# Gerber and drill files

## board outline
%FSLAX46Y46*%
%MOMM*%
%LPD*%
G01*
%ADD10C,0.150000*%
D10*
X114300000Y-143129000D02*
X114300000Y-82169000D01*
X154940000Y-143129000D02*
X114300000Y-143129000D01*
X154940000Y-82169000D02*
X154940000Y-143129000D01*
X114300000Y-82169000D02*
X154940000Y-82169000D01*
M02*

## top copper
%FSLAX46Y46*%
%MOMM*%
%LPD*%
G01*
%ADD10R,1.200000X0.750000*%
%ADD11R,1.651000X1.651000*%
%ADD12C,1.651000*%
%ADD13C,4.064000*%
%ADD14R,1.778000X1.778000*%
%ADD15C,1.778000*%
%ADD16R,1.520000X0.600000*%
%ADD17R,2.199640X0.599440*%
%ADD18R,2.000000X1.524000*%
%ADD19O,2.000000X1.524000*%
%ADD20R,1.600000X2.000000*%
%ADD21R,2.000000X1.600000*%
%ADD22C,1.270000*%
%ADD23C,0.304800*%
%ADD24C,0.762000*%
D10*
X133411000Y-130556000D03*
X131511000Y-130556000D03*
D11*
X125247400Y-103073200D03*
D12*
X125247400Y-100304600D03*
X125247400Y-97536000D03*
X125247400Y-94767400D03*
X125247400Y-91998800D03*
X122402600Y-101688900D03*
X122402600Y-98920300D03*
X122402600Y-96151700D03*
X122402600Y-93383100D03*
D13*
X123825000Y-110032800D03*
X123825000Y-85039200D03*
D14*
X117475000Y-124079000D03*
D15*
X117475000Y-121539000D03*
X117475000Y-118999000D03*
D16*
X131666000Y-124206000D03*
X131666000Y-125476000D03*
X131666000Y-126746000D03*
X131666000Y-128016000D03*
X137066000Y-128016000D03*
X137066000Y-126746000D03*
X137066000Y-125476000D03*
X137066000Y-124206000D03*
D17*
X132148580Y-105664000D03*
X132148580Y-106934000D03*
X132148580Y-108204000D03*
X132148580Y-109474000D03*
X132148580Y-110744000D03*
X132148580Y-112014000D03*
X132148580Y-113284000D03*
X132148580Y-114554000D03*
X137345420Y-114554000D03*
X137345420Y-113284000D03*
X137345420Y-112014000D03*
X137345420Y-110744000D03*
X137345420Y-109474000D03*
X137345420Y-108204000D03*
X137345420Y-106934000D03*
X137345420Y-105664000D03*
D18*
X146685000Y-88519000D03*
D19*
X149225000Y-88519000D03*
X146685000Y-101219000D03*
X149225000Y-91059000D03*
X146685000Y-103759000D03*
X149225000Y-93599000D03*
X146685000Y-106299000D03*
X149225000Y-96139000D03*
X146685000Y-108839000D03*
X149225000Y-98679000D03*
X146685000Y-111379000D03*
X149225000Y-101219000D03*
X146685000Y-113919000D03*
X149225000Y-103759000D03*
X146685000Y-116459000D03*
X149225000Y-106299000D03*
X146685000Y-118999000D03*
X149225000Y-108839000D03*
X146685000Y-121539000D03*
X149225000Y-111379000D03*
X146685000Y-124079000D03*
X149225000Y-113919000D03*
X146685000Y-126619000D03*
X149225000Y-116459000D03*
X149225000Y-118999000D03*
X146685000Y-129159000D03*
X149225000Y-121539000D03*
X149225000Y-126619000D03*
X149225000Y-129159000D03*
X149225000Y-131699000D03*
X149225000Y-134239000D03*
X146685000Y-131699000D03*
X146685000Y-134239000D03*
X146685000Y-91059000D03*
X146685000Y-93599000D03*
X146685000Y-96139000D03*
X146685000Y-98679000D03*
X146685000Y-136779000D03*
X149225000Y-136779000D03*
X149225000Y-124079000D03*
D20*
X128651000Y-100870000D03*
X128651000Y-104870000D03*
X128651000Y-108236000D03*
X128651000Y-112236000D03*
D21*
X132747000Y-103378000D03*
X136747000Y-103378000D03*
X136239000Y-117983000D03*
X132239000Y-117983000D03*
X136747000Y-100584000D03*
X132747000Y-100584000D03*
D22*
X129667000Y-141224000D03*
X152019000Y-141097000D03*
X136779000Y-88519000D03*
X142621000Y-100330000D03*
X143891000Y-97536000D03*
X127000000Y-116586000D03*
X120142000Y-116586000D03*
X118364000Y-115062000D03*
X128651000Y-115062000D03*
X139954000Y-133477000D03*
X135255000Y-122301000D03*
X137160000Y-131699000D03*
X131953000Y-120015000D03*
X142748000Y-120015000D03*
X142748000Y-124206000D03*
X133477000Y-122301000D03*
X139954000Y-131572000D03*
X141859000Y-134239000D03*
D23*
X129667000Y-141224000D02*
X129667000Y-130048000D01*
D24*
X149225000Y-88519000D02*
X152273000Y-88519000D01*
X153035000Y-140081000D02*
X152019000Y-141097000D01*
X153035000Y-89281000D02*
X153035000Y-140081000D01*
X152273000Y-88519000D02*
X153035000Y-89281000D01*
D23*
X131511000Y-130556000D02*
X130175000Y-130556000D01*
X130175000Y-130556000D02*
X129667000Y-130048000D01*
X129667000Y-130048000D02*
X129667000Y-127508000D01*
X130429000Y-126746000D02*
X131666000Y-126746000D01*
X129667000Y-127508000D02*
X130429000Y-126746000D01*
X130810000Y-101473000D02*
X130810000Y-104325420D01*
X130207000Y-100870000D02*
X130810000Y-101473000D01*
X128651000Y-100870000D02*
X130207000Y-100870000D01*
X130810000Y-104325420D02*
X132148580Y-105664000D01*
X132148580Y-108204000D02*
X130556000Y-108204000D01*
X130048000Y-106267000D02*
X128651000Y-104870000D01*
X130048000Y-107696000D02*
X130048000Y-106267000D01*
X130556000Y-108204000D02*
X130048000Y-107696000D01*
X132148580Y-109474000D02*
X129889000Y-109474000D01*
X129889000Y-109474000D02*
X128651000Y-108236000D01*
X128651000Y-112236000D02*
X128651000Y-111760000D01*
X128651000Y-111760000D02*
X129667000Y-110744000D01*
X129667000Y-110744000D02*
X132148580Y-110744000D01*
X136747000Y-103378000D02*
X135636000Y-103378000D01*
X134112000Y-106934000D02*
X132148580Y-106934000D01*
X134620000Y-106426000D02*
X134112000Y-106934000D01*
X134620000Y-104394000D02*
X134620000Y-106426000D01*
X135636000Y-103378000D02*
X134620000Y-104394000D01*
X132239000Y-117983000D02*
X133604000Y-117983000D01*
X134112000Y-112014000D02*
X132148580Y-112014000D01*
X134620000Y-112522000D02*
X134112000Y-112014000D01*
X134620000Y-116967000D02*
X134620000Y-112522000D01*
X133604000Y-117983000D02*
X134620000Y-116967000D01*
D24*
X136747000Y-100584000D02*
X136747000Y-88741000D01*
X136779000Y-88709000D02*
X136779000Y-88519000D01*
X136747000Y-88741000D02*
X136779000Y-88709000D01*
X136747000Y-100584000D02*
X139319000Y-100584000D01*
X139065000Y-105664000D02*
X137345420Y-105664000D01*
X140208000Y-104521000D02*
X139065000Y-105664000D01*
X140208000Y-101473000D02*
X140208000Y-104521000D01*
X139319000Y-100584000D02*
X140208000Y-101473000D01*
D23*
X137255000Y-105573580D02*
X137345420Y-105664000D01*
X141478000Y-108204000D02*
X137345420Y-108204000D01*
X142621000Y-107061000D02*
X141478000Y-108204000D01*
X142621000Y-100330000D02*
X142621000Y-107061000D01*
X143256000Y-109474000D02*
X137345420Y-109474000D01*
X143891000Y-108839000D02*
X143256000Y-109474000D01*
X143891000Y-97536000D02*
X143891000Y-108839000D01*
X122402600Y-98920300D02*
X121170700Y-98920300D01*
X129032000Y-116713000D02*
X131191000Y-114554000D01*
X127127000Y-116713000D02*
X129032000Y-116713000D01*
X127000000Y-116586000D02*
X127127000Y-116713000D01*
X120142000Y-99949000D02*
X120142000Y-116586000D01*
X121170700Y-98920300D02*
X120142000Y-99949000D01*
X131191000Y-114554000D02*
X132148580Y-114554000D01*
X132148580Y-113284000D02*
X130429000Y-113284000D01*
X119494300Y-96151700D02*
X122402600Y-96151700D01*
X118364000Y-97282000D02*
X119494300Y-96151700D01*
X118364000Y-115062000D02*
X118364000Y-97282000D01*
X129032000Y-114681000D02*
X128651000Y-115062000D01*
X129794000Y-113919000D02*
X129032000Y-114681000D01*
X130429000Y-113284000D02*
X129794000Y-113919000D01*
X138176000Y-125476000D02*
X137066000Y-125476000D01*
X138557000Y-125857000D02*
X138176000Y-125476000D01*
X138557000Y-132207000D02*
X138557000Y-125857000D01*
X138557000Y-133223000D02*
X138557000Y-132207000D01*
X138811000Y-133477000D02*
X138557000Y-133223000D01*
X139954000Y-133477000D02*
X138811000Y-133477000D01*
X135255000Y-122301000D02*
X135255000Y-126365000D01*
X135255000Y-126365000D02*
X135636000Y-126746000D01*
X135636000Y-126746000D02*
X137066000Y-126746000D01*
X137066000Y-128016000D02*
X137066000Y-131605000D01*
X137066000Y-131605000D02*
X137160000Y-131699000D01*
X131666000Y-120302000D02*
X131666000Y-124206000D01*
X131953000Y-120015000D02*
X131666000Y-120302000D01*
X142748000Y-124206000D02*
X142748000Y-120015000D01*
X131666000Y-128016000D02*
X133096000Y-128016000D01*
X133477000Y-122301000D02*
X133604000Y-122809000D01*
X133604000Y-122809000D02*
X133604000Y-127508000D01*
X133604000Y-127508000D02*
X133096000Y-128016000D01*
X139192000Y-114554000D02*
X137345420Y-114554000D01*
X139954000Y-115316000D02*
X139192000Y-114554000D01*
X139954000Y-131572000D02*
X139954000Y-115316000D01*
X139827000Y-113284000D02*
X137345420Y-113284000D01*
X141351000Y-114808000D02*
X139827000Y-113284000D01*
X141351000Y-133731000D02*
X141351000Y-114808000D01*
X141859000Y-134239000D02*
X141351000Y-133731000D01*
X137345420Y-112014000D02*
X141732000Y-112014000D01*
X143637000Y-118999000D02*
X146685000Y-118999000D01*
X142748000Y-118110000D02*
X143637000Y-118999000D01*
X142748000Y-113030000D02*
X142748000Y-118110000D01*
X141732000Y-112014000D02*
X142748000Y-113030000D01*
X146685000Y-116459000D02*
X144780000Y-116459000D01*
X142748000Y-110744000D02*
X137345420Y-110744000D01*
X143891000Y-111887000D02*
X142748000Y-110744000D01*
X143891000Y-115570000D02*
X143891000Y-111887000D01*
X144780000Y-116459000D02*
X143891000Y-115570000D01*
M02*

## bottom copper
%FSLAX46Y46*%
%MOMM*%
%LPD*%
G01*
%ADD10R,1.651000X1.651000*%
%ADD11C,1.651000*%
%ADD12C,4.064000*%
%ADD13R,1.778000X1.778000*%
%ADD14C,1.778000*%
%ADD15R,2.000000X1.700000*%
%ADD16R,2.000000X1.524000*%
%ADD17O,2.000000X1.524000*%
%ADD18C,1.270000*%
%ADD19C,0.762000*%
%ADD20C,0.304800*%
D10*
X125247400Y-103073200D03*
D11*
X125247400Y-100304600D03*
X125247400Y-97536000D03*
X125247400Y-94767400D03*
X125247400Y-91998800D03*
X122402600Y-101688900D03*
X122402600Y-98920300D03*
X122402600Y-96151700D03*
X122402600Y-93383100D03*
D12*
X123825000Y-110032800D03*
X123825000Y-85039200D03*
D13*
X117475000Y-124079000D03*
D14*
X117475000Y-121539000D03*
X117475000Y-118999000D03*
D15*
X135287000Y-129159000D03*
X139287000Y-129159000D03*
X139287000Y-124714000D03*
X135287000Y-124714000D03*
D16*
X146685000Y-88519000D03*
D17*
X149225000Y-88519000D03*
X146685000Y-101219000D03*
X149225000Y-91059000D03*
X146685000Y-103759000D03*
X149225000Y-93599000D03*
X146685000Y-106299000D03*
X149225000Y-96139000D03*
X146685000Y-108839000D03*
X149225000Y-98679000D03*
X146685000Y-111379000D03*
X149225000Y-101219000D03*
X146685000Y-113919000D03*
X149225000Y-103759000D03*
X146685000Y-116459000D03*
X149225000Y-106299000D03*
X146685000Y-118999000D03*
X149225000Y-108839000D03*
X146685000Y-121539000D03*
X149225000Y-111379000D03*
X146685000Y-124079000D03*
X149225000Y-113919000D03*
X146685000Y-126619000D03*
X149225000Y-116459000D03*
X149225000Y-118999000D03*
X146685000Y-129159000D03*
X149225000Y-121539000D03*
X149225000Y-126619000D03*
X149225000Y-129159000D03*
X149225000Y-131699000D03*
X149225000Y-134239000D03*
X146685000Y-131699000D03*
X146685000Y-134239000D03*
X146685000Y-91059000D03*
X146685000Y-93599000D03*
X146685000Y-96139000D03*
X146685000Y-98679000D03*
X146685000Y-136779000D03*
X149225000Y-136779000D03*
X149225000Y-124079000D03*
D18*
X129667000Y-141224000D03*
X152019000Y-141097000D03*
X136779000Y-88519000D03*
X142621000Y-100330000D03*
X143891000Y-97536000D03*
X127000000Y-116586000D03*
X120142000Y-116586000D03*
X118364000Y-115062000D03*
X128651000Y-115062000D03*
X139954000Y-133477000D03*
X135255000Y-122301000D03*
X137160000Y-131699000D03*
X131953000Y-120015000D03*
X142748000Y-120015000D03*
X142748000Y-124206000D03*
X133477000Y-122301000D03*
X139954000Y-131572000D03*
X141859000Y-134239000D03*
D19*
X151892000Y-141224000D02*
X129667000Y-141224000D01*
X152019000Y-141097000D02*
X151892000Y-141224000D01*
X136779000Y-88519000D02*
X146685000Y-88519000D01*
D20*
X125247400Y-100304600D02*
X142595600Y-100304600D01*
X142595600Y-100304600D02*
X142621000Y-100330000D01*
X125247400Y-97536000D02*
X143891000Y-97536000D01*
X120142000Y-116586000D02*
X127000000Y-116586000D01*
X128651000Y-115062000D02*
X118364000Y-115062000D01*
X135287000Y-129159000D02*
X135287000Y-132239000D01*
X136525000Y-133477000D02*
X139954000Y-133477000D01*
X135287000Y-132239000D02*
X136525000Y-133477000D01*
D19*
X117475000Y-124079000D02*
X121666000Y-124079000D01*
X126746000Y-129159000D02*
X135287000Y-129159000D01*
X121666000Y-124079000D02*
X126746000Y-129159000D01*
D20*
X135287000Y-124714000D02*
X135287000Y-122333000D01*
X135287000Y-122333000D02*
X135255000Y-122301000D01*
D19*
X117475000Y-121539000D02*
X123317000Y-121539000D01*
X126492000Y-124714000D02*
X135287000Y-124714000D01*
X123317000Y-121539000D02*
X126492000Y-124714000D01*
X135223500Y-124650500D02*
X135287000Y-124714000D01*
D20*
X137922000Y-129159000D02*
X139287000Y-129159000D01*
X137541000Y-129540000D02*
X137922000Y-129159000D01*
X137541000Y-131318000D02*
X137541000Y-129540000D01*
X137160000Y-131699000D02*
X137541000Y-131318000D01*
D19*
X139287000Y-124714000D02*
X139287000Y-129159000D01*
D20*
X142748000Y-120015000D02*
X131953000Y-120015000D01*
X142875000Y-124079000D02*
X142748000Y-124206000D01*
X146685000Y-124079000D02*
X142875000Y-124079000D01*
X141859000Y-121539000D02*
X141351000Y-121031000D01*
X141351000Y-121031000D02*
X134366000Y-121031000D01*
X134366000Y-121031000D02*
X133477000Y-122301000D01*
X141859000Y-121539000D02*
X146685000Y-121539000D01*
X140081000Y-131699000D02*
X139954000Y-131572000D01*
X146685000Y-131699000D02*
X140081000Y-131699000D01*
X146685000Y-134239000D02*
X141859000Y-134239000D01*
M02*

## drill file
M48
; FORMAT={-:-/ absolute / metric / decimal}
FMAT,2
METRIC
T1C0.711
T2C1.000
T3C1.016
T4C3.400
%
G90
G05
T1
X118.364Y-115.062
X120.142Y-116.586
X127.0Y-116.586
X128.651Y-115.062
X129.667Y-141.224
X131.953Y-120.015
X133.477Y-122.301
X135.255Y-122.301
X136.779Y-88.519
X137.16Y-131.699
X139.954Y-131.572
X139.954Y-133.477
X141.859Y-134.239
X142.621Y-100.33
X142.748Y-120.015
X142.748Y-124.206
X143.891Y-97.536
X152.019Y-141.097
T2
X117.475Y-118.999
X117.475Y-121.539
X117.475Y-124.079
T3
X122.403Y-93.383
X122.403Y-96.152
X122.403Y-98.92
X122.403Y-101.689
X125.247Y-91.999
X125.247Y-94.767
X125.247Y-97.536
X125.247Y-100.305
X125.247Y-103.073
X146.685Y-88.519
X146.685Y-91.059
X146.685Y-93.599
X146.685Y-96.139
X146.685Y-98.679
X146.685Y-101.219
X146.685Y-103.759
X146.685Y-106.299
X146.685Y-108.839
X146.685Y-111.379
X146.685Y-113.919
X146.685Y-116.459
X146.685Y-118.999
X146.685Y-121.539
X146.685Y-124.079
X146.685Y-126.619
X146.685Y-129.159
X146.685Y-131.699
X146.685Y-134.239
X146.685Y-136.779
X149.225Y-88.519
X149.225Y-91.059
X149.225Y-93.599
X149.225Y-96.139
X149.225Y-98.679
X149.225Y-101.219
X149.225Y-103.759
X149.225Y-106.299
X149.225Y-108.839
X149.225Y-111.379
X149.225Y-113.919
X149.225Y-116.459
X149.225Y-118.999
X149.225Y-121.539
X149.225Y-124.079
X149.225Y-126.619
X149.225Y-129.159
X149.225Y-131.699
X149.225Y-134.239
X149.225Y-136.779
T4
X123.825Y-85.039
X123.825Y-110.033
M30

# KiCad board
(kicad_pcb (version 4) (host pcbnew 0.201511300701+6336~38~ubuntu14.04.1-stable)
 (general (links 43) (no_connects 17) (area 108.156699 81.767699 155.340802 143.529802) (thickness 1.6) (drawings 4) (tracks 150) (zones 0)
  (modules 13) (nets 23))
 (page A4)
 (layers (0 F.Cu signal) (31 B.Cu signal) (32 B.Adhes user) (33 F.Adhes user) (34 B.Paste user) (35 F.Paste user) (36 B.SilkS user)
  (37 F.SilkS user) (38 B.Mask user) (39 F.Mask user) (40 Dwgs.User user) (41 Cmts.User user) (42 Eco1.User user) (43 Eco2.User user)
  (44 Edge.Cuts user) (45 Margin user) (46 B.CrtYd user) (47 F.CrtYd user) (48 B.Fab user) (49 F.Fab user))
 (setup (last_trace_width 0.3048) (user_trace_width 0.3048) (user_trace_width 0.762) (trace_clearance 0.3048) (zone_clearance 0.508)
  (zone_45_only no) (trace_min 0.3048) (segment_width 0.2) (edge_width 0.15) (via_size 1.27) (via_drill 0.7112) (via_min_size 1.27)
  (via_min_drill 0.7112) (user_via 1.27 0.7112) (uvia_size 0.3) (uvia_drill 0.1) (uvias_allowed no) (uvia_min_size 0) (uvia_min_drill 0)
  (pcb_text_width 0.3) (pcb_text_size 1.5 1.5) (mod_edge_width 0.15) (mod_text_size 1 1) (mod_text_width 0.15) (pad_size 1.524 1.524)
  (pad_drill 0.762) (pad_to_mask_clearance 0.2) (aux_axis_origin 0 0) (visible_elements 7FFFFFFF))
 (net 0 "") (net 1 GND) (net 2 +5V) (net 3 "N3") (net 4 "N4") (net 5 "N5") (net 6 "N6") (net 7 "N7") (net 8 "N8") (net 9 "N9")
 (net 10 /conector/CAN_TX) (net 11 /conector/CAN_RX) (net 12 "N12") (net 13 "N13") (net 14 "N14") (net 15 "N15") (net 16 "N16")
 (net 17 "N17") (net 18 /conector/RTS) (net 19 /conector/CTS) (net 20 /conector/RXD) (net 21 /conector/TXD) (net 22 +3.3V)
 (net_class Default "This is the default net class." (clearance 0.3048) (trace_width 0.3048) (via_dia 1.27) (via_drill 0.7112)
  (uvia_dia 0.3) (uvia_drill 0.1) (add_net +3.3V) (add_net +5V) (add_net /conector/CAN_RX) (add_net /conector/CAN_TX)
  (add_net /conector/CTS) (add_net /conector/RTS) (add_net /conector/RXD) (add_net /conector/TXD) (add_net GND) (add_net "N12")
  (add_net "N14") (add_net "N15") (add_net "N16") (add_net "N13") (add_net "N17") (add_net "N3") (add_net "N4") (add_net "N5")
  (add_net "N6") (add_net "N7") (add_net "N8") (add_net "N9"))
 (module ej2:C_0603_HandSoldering (layer F.Cu) (at 132.461 130.556 180)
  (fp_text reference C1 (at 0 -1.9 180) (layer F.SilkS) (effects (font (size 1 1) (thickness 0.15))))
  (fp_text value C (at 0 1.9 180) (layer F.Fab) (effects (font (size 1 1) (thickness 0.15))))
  (pad 1 smd rect (at -0.95 0 180) (size 1.2 0.75) (layers F.Cu F.Paste F.Mask) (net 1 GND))
  (pad 2 smd rect (at 0.95 0 180) (size 1.2 0.75) (layers F.Cu F.Paste F.Mask) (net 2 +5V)))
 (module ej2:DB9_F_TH (layer F.Cu) (at 123.825 97.536 90)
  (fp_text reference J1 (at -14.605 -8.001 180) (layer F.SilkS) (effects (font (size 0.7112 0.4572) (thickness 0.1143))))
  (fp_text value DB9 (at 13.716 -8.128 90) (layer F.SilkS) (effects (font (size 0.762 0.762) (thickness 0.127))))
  (pad 1 thru_hole rect (at -5.5372 1.4224 90) (size 1.651 1.651) (drill 1.016) (layers *.Cu *.Mask))
  (pad 2 thru_hole circle (at -2.7686 1.4224 90) (size 1.651 1.651) (drill 1.016) (layers *.Cu *.Mask) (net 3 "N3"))
  (pad 3 thru_hole circle (at 0 1.4224 90) (size 1.651 1.651) (drill 1.016) (layers *.Cu *.Mask) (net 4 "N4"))
  (pad 4 thru_hole circle (at 2.7686 1.4224 90) (size 1.651 1.651) (drill 1.016) (layers *.Cu *.Mask))
  (pad 5 thru_hole circle (at 5.5372 1.4224 90) (size 1.651 1.651) (drill 1.016) (layers *.Cu *.Mask))
  (pad 6 thru_hole circle (at -4.1529 -1.4224 90) (size 1.651 1.651) (drill 1.016) (layers *.Cu *.Mask))
  (pad 7 thru_hole circle (at -1.3843 -1.4224 90) (size 1.651 1.651) (drill 1.016) (layers *.Cu *.Mask) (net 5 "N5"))
  (pad 8 thru_hole circle (at 1.3843 -1.4224 90) (size 1.651 1.651) (drill 1.016) (layers *.Cu *.Mask) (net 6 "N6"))
  (pad 9 thru_hole circle (at 4.1529 -1.4224 90) (size 1.651 1.651) (drill 1.016) (layers *.Cu *.Mask))
  (pad 10 thru_hole circle (at -12.4968 0 90) (size 4.064 4.064) (drill 3.4) (layers *.Cu *.Mask))
  (pad 11 thru_hole circle (at 12.4968 0 90) (size 4.064 4.064) (drill 3.4) (layers *.Cu *.Mask)))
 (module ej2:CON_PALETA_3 (layer F.Cu) (at 117.475 121.539 90)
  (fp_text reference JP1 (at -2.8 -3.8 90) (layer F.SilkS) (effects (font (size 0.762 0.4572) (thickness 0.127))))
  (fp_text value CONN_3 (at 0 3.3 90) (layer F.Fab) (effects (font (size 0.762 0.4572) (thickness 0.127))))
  (pad 1 thru_hole rect (at -2.54 0 90) (size 1.778 1.778) (drill 1) (layers *.Cu *.Mask) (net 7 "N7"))
  (pad 2 thru_hole circle (at 0 0 90) (size 1.778 1.778) (drill 1) (layers *.Cu *.Mask) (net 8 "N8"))
  (pad 3 thru_hole circle (at 2.54 0 90) (size 1.778 1.778) (drill 1) (layers *.Cu *.Mask) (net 1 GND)))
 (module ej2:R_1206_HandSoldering (layer B.Cu) (at 137.287 129.159)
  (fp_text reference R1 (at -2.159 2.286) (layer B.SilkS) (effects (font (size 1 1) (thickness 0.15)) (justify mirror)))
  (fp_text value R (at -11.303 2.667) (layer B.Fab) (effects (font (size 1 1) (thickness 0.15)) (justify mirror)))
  (pad 1 smd rect (at -2 0) (size 2 1.7) (layers B.Cu B.Paste B.Mask) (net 7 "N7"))
  (pad 2 smd rect (at 2 0) (size 2 1.7) (layers B.Cu B.Paste B.Mask) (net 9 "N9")))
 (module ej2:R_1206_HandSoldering (layer B.Cu) (at 137.287 124.714 180)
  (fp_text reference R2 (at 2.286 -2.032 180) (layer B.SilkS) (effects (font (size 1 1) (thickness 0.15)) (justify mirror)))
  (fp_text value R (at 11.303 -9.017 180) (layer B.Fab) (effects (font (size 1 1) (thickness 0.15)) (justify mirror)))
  (pad 1 smd rect (at -2 0 180) (size 2 1.7) (layers B.Cu B.Paste B.Mask) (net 9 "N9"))
  (pad 2 smd rect (at 2 0 180) (size 2 1.7) (layers B.Cu B.Paste B.Mask) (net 8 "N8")))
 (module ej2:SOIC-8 (layer F.Cu) (at 134.366 126.111)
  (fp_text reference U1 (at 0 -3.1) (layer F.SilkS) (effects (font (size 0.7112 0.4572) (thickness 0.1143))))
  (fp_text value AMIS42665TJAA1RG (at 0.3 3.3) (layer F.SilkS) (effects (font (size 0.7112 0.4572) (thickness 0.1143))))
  (pad 1 smd rect (at -2.7 -1.905 270) (size 0.6 1.52) (layers F.Cu F.Paste F.Mask) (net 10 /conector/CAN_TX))
  (pad 2 smd rect (at -2.7 -0.635 270) (size 0.6 1.52) (layers F.Cu F.Paste F.Mask) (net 1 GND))
  (pad 3 smd rect (at -2.7 0.635 270) (size 0.6 1.52) (layers F.Cu F.Paste F.Mask) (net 2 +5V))
  (pad 4 smd rect (at -2.7 1.905 270) (size 0.6 1.52) (layers F.Cu F.Paste F.Mask) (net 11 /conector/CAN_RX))
  (pad 5 smd rect (at 2.7 1.905 270) (size 0.6 1.52) (layers F.Cu F.Paste F.Mask) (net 9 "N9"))
  (pad 6 smd rect (at 2.7 0.635 270) (size 0.6 1.52) (layers F.Cu F.Paste F.Mask) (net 8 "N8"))
  (pad 7 smd rect (at 2.7 -0.635 270) (size 0.6 1.52) (layers F.Cu F.Paste F.Mask) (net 7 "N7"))
  (pad 8 smd rect (at 2.7 -1.905 270) (size 0.6 1.52) (layers F.Cu F.Paste F.Mask) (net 1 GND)))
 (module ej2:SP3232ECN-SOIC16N (layer F.Cu) (at 134.747 110.109 270)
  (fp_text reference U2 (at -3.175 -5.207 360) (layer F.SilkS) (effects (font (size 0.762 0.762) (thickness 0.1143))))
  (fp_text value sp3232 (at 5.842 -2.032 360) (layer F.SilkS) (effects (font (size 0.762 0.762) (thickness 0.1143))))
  (pad 1 smd rect (at -4.445 2.59842 270) (size 0.59944 2.19964) (layers F.Cu F.Paste F.Mask) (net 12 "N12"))
  (pad 2 smd rect (at -3.175 2.59842 270) (size 0.59944 2.19964) (layers F.Cu F.Paste F.Mask) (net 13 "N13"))
  (pad 3 smd rect (at -1.905 2.59842 270) (size 0.59944 2.19964) (layers F.Cu F.Paste F.Mask) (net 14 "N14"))
  (pad 4 smd rect (at -0.635 2.59842 270) (size 0.59944 2.19964) (layers F.Cu F.Paste F.Mask) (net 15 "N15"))
  (pad 5 smd rect (at 0.635 2.59842 270) (size 0.59944 2.19964) (layers F.Cu F.Paste F.Mask) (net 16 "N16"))
  (pad 6 smd rect (at 1.905 2.59842 270) (size 0.59944 2.19964) (layers F.Cu F.Paste F.Mask) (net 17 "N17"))
  (pad 7 smd rect (at 3.175 2.59842 270) (size 0.59944 2.19964) (layers F.Cu F.Paste F.Mask) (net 6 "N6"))
  (pad 8 smd rect (at 4.445 2.59842 270) (size 0.59944 2.19964) (layers F.Cu F.Paste F.Mask) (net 5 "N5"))
  (pad 9 smd rect (at 4.445 -2.59842 270) (size 0.59944 2.19964) (layers F.Cu F.Paste F.Mask) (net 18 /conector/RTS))
  (pad 10 smd rect (at 3.175 -2.59842 270) (size 0.59944 2.19964) (layers F.Cu F.Paste F.Mask) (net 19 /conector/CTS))
  (pad 11 smd rect (at 1.905 -2.59842 270) (size 0.59944 2.19964) (layers F.Cu F.Paste F.Mask) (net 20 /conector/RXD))
  (pad 12 smd rect (at 0.635 -2.59842 270) (size 0.59944 2.19964) (layers F.Cu F.Paste F.Mask) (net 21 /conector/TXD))
  (pad 13 smd rect (at -0.635 -2.59842 270) (size 0.59944 2.19964) (layers F.Cu F.Paste F.Mask) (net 4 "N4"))
  (pad 14 smd rect (at -1.905 -2.59842 270) (size 0.59944 2.19964) (layers F.Cu F.Paste F.Mask) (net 3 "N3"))
  (pad 15 smd rect (at -3.175 -2.59842 270) (size 0.59944 2.19964) (layers F.Cu F.Paste F.Mask) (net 1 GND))
  (pad 16 smd rect (at -4.445 -2.59842 270) (size 0.59944 2.19964) (layers F.Cu F.Paste F.Mask) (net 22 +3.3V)))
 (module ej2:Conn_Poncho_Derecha (layer F.Cu) (at 146.685 88.519)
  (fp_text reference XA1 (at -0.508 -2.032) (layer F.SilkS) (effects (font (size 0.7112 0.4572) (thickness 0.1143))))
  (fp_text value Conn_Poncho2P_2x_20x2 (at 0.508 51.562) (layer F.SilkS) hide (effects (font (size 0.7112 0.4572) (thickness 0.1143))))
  (pad 1 thru_hole rect (at 0 0 270) (size 1.524 2) (drill 1.016) (layers *.Cu *.Mask) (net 22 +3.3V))
  (pad 2 thru_hole oval (at 2.54 0 270) (size 1.524 2) (drill 1.016) (layers *.Cu *.Mask) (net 2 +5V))
  (pad 11 thru_hole oval (at 0 12.7 270) (size 1.524 2) (drill 1.016) (layers *.Cu *.Mask))
  (pad 4 thru_hole oval (at 2.54 2.54 270) (size 1.524 2) (drill 1.016) (layers *.Cu *.Mask) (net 1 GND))
  (pad 13 thru_hole oval (at 0 15.24 270) (size 1.524 2) (drill 1.016) (layers *.Cu *.Mask))
  (pad 6 thru_hole oval (at 2.54 5.08 270) (size 1.524 2) (drill 1.016) (layers *.Cu *.Mask))
  (pad 15 thru_hole oval (at 0 17.78 270) (size 1.524 2) (drill 1.016) (layers *.Cu *.Mask))
  (pad 8 thru_hole oval (at 2.54 7.62 270) (size 1.524 2) (drill 1.016) (layers *.Cu *.Mask))
  (pad 17 thru_hole oval (at 0 20.32 270) (size 1.524 2) (drill 1.016) (layers *.Cu *.Mask))
  (pad 10 thru_hole oval (at 2.54 10.16 270) (size 1.524 2) (drill 1.016) (layers *.Cu *.Mask))
  (pad 19 thru_hole oval (at 0 22.86 270) (size 1.524 2) (drill 1.016) (layers *.Cu *.Mask))
  (pad 12 thru_hole oval (at 2.54 12.7 270) (size 1.524 2) (drill 1.016) (layers *.Cu *.Mask))
  (pad 21 thru_hole oval (at 0 25.4 270) (size 1.524 2) (drill 1.016) (layers *.Cu *.Mask))
  (pad 14 thru_hole oval (at 2.54 15.24 270) (size 1.524 2) (drill 1.016) (layers *.Cu *.Mask))
  (pad 23 thru_hole oval (at 0 27.94 270) (size 1.524 2) (drill 1.016) (layers *.Cu *.Mask) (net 21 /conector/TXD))
  (pad 16 thru_hole oval (at 2.54 17.78 270) (size 1.524 2) (drill 1.016) (layers *.Cu *.Mask))
  (pad 25 thru_hole oval (at 0 30.48 270) (size 1.524 2) (drill 1.016) (layers *.Cu *.Mask) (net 20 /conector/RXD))
  (pad 18 thru_hole oval (at 2.54 20.32 270) (size 1.524 2) (drill 1.016) (layers *.Cu *.Mask))
  (pad 27 thru_hole oval (at 0 33.02 270) (size 1.524 2) (drill 1.016) (layers *.Cu *.Mask) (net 11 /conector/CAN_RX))
  (pad 20 thru_hole oval (at 2.54 22.86 270) (size 1.524 2) (drill 1.016) (layers *.Cu *.Mask) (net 1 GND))
  (pad 29 thru_hole oval (at 0 35.56 270) (size 1.524 2) (drill 1.016) (layers *.Cu *.Mask) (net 10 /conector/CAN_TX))
  (pad 22 thru_hole oval (at 2.54 25.4 270) (size 1.524 2) (drill 1.016) (layers *.Cu *.Mask) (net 1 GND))
  (pad 31 thru_hole oval (at 0 38.1 270) (size 1.524 2) (drill 1.016) (layers *.Cu *.Mask))
  (pad 24 thru_hole oval (at 2.54 27.94 270) (size 1.524 2) (drill 1.016) (layers *.Cu *.Mask) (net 1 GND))
  (pad 26 thru_hole oval (at 2.54 30.48 270) (size 1.524 2) (drill 1.016) (layers *.Cu *.Mask) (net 1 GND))
  (pad 33 thru_hole oval (at 0 40.64 270) (size 1.524 2) (drill 1.016) (layers *.Cu *.Mask))
  (pad 28 thru_hole oval (at 2.54 33.02 270) (size 1.524 2) (drill 1.016) (layers *.Cu *.Mask) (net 1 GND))
  (pad 32 thru_hole oval (at 2.54 38.1 270) (size 1.524 2) (drill 1.016) (layers *.Cu *.Mask) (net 1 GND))
  (pad 34 thru_hole oval (at 2.54 40.64 270) (size 1.524 2) (drill 1.016) (layers *.Cu *.Mask))
  (pad 36 thru_hole oval (at 2.54 43.18 270) (size 1.524 2) (drill 1.016) (layers *.Cu *.Mask))
  (pad 38 thru_hole oval (at 2.54 45.72 270) (size 1.524 2) (drill 1.016) (layers *.Cu *.Mask) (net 1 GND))
  (pad 35 thru_hole oval (at 0 43.18 270) (size 1.524 2) (drill 1.016) (layers *.Cu *.Mask) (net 18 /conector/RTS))
  (pad 37 thru_hole oval (at 0 45.72 270) (size 1.524 2) (drill 1.016) (layers *.Cu *.Mask) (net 19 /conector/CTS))
  (pad 3 thru_hole oval (at 0 2.54 270) (size 1.524 2) (drill 1.016) (layers *.Cu *.Mask))
  (pad 5 thru_hole oval (at 0 5.08 270) (size 1.524 2) (drill 1.016) (layers *.Cu *.Mask))
  (pad 7 thru_hole oval (at 0 7.62 270) (size 1.524 2) (drill 1.016) (layers *.Cu *.Mask))
  (pad 9 thru_hole oval (at 0 10.16 270) (size 1.524 2) (drill 1.016) (layers *.Cu *.Mask))
  (pad 39 thru_hole oval (at 0 48.26 270) (size 1.524 2) (drill 1.016) (layers *.Cu *.Mask))
  (pad 40 thru_hole oval (at 2.54 48.26 270) (size 1.524 2) (drill 1.016) (layers *.Cu *.Mask) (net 1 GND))
  (pad 30 thru_hole oval (at 2.54 35.56 270) (size 1.524 2) (drill 1.016) (layers *.Cu *.Mask) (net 1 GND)))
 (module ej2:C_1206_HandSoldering (layer F.Cu) (at 128.651 102.87 270)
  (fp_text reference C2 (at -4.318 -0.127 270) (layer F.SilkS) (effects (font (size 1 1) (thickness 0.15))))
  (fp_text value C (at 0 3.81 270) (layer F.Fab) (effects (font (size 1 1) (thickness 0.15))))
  (pad 1 smd rect (at -2 0 270) (size 2 1.6) (layers F.Cu F.Paste F.Mask) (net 12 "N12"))
  (pad 2 smd rect (at 2 0 270) (size 2 1.6) (layers F.Cu F.Paste F.Mask) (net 14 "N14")))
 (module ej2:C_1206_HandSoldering (layer F.Cu) (at 128.651 110.236 270)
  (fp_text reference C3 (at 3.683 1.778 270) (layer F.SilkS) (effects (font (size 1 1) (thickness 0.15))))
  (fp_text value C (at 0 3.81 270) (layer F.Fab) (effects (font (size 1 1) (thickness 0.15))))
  (pad 1 smd rect (at -2 0 270) (size 2 1.6) (layers F.Cu F.Paste F.Mask) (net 15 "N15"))
  (pad 2 smd rect (at 2 0 270) (size 2 1.6) (layers F.Cu F.Paste F.Mask) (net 16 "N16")))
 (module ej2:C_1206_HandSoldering (layer F.Cu) (at 134.747 103.378)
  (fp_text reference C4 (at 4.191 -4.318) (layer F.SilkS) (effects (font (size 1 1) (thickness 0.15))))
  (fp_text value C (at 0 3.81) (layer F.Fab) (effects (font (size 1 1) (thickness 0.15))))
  (pad 1 smd rect (at -2 0) (size 2 1.6) (layers F.Cu F.Paste F.Mask) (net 1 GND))
  (pad 2 smd rect (at 2 0) (size 2 1.6) (layers F.Cu F.Paste F.Mask) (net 13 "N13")))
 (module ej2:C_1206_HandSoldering (layer F.Cu) (at 134.239 117.983 180)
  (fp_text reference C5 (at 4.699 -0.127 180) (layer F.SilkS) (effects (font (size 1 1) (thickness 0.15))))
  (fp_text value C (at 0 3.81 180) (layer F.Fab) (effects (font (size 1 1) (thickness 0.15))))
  (pad 1 smd rect (at -2 0 180) (size 2 1.6) (layers F.Cu F.Paste F.Mask) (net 1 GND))
  (pad 2 smd rect (at 2 0 180) (size 2 1.6) (layers F.Cu F.Paste F.Mask) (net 17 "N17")))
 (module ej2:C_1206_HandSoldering (layer F.Cu) (at 134.747 100.584 180)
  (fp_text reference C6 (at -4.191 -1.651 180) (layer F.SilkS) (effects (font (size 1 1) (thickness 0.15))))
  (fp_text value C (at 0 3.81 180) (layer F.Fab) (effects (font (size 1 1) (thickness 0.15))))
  (pad 1 smd rect (at -2 0 180) (size 2 1.6) (layers F.Cu F.Paste F.Mask) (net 22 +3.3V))
  (pad 2 smd rect (at 2 0 180) (size 2 1.6) (layers F.Cu F.Paste F.Mask) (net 1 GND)))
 (gr_line (start 114.3 143.129) (end 114.3 82.169) (angle 90) (layer Edge.Cuts) (width 0.15))
 (gr_line (start 154.94 143.129) (end 114.3 143.129) (angle 90) (layer Edge.Cuts) (width 0.15))
 (gr_line (start 154.94 82.169) (end 154.94 143.129) (angle 90) (layer Edge.Cuts) (width 0.15))
 (gr_line (start 114.3 82.169) (end 154.94 82.169) (angle 90) (layer Edge.Cuts) (width 0.15))
 (segment (start 129.667 141.224) (end 129.667 130.048) (width 0.3048) (layer F.Cu) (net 2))
 (segment (start 149.225 88.519) (end 152.273 88.519) (width 0.762) (layer F.Cu) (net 2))
 (via (at 129.667 141.224) (size 1.27) (drill 0.7112) (layers F.Cu B.Cu) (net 2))
 (segment (start 151.892 141.224) (end 129.667 141.224) (width 0.762) (layer B.Cu) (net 2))
 (segment (start 152.019 141.097) (end 151.892 141.224) (width 0.762) (layer B.Cu) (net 2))
 (via (at 152.019 141.097) (size 1.27) (drill 0.7112) (layers F.Cu B.Cu) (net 2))
 (segment (start 153.035 140.081) (end 152.019 141.097) (width 0.762) (layer F.Cu) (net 2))
 (segment (start 153.035 89.281) (end 153.035 140.081) (width 0.762) (layer F.Cu) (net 2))
 (segment (start 152.273 88.519) (end 153.035 89.281) (width 0.762) (layer F.Cu) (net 2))
 (segment (start 131.511 130.556) (end 130.175 130.556) (width 0.3048) (layer F.Cu) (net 2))
 (segment (start 130.175 130.556) (end 129.667 130.048) (width 0.3048) (layer F.Cu) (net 2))
 (segment (start 129.667 130.048) (end 129.667 127.508) (width 0.3048) (layer F.Cu) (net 2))
 (segment (start 130.429 126.746) (end 131.666 126.746) (width 0.3048) (layer F.Cu) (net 2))
 (segment (start 129.667 127.508) (end 130.429 126.746) (width 0.3048) (layer F.Cu) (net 2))
 (segment (start 130.81 101.473) (end 130.81 104.32542) (width 0.3048) (layer F.Cu) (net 12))
 (segment (start 130.207 100.87) (end 130.81 101.473) (width 0.3048) (layer F.Cu) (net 12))
 (segment (start 128.651 100.87) (end 130.207 100.87) (width 0.3048) (layer F.Cu) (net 12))
 (segment (start 130.81 104.32542) (end 132.14858 105.664) (width 0.3048) (layer F.Cu) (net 12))
 (segment (start 132.14858 108.204) (end 130.556 108.204) (width 0.3048) (layer F.Cu) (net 14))
 (segment (start 130.048 106.267) (end 128.651 104.87) (width 0.3048) (layer F.Cu) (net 14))
 (segment (start 130.048 107.696) (end 130.048 106.267) (width 0.3048) (layer F.Cu) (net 14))
 (segment (start 130.556 108.204) (end 130.048 107.696) (width 0.3048) (layer F.Cu) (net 14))
 (segment (start 132.14858 109.474) (end 129.889 109.474) (width 0.3048) (layer F.Cu) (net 15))
 (segment (start 129.889 109.474) (end 128.651 108.236) (width 0.3048) (layer F.Cu) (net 15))
 (segment (start 128.651 112.236) (end 128.651 111.76) (width 0.3048) (layer F.Cu) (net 16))
 (segment (start 128.651 111.76) (end 129.667 110.744) (width 0.3048) (layer F.Cu) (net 16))
 (segment (start 129.667 110.744) (end 132.14858 110.744) (width 0.3048) (layer F.Cu) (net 16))
 (segment (start 136.747 103.378) (end 135.636 103.378) (width 0.3048) (layer F.Cu) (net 13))
 (segment (start 134.112 106.934) (end 132.14858 106.934) (width 0.3048) (layer F.Cu) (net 13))
 (segment (start 134.62 106.426) (end 134.112 106.934) (width 0.3048) (layer F.Cu) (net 13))
 (segment (start 134.62 104.394) (end 134.62 106.426) (width 0.3048) (layer F.Cu) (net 13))
 (segment (start 135.636 103.378) (end 134.62 104.394) (width 0.3048) (layer F.Cu) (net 13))
 (segment (start 132.239 117.983) (end 133.604 117.983) (width 0.3048) (layer F.Cu) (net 17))
 (segment (start 134.112 112.014) (end 132.14858 112.014) (width 0.3048) (layer F.Cu) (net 17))
 (segment (start 134.62 112.522) (end 134.112 112.014) (width 0.3048) (layer F.Cu) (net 17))
 (segment (start 134.62 116.967) (end 134.62 112.522) (width 0.3048) (layer F.Cu) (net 17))
 (segment (start 133.604 117.983) (end 134.62 116.967) (width 0.3048) (layer F.Cu) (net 17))
 (segment (start 136.747 100.584) (end 136.747 88.741) (width 0.762) (layer F.Cu) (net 22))
 (segment (start 136.779 88.519) (end 146.685 88.519) (width 0.762) (layer B.Cu) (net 22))
 (via (at 136.779 88.519) (size 1.27) (drill 0.7112) (layers F.Cu B.Cu) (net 22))
 (segment (start 136.779 88.709) (end 136.779 88.519) (width 0.762) (layer F.Cu) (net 22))
 (segment (start 136.747 88.741) (end 136.779 88.709) (width 0.762) (layer F.Cu) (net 22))
 (segment (start 136.747 100.584) (end 139.319 100.584) (width 0.762) (layer F.Cu) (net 22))
 (segment (start 139.065 105.664) (end 137.34542 105.664) (width 0.762) (layer F.Cu) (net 22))
 (segment (start 140.208 104.521) (end 139.065 105.664) (width 0.762) (layer F.Cu) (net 22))
 (segment (start 140.208 101.473) (end 140.208 104.521) (width 0.762) (layer F.Cu) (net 22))
 (segment (start 139.319 100.584) (end 140.208 101.473) (width 0.762) (layer F.Cu) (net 22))
 (segment (start 137.255 105.57358) (end 137.34542 105.664) (width 0.3048) (layer F.Cu) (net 22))
 (segment (start 125.2474 100.3046) (end 142.5956 100.3046) (width 0.3048) (layer B.Cu) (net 3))
 (segment (start 141.478 108.204) (end 137.34542 108.204) (width 0.3048) (layer F.Cu) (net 3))
 (segment (start 142.621 107.061) (end 141.478 108.204) (width 0.3048) (layer F.Cu) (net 3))
 (segment (start 142.621 100.33) (end 142.621 107.061) (width 0.3048) (layer F.Cu) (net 3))
 (via (at 142.621 100.33) (size 1.27) (drill 0.7112) (layers F.Cu B.Cu) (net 3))
 (segment (start 142.5956 100.3046) (end 142.621 100.33) (width 0.3048) (layer B.Cu) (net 3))
 (segment (start 125.2474 97.536) (end 143.891 97.536) (width 0.3048) (layer B.Cu) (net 4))
 (segment (start 143.256 109.474) (end 137.34542 109.474) (width 0.3048) (layer F.Cu) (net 4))
 (segment (start 143.891 108.839) (end 143.256 109.474) (width 0.3048) (layer F.Cu) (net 4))
 (segment (start 143.891 97.536) (end 143.891 108.839) (width 0.3048) (layer F.Cu) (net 4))
 (via (at 143.891 97.536) (size 1.27) (drill 0.7112) (layers F.Cu B.Cu) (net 4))
 (segment (start 122.4026 98.9203) (end 121.1707 98.9203) (width 0.3048) (layer F.Cu) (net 5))
 (segment (start 129.032 116.713) (end 131.191 114.554) (width 0.3048) (layer F.Cu) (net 5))
 (segment (start 127.127 116.713) (end 129.032 116.713) (width 0.3048) (layer F.Cu) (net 5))
 (segment (start 127 116.586) (end 127.127 116.713) (width 0.3048) (layer F.Cu) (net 5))
 (via (at 127 116.586) (size 1.27) (drill 0.7112) (layers F.Cu B.Cu) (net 5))
 (segment (start 120.142 116.586) (end 127 116.586) (width 0.3048) (layer B.Cu) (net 5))
 (via (at 120.142 116.586) (size 1.27) (drill 0.7112) (layers F.Cu B.Cu) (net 5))
 (segment (start 120.142 99.949) (end 120.142 116.586) (width 0.3048) (layer F.Cu) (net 5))
 (segment (start 121.1707 98.9203) (end 120.142 99.949) (width 0.3048) (layer F.Cu) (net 5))
 (segment (start 131.191 114.554) (end 132.14858 114.554) (width 0.3048) (layer F.Cu) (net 5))
 (segment (start 132.14858 113.284) (end 130.429 113.284) (width 0.3048) (layer F.Cu) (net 6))
 (segment (start 119.4943 96.1517) (end 122.4026 96.1517) (width 0.3048) (layer F.Cu) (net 6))
 (segment (start 118.364 97.282) (end 119.4943 96.1517) (width 0.3048) (layer F.Cu) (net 6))
 (segment (start 118.364 115.062) (end 118.364 97.282) (width 0.3048) (layer F.Cu) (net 6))
 (via (at 118.364 115.062) (size 1.27) (drill 0.7112) (layers F.Cu B.Cu) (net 6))
 (segment (start 128.651 115.062) (end 118.364 115.062) (width 0.3048) (layer B.Cu) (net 6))
 (via (at 128.651 115.062) (size 1.27) (drill 0.7112) (layers F.Cu B.Cu) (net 6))
 (segment (start 129.032 114.681) (end 128.651 115.062) (width 0.3048) (layer F.Cu) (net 6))
 (segment (start 129.794 113.919) (end 129.032 114.681) (width 0.3048) (layer F.Cu) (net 6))
 (segment (start 130.429 113.284) (end 129.794 113.919) (width 0.3048) (layer F.Cu) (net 6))
 (segment (start 135.287 129.159) (end 135.287 132.239) (width 0.3048) (layer B.Cu) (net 7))
 (segment (start 138.176 125.476) (end 137.066 125.476) (width 0.3048) (layer F.Cu) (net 7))
 (segment (start 138.557 125.857) (end 138.176 125.476) (width 0.3048) (layer F.Cu) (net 7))
 (segment (start 138.557 132.207) (end 138.557 125.857) (width 0.3048) (layer F.Cu) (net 7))
 (segment (start 138.557 133.223) (end 138.557 132.207) (width 0.3048) (layer F.Cu) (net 7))
 (segment (start 138.811 133.477) (end 138.557 133.223) (width 0.3048) (layer F.Cu) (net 7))
 (segment (start 139.954 133.477) (end 138.811 133.477) (width 0.3048) (layer F.Cu) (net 7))
 (via (at 139.954 133.477) (size 1.27) (drill 0.7112) (layers F.Cu B.Cu) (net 7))
 (segment (start 136.525 133.477) (end 139.954 133.477) (width 0.3048) (layer B.Cu) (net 7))
 (segment (start 135.287 132.239) (end 136.525 133.477) (width 0.3048) (layer B.Cu) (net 7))
 (segment (start 117.475 124.079) (end 121.666 124.079) (width 0.762) (layer B.Cu) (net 7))
 (segment (start 126.746 129.159) (end 135.287 129.159) (width 0.762) (layer B.Cu) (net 7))
 (segment (start 121.666 124.079) (end 126.746 129.159) (width 0.762) (layer B.Cu) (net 7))
 (segment (start 135.287 124.714) (end 135.287 122.333) (width 0.3048) (layer B.Cu) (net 8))
 (segment (start 135.287 122.333) (end 135.255 122.301) (width 0.3048) (layer B.Cu) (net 8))
 (via (at 135.255 122.301) (size 1.27) (drill 0.7112) (layers F.Cu B.Cu) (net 8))
 (segment (start 135.255 122.301) (end 135.255 126.365) (width 0.3048) (layer F.Cu) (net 8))
 (segment (start 135.255 126.365) (end 135.636 126.746) (width 0.3048) (layer F.Cu) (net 8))
 (segment (start 135.636 126.746) (end 137.066 126.746) (width 0.3048) (layer F.Cu) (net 8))
 (segment (start 117.475 121.539) (end 123.317 121.539) (width 0.762) (layer B.Cu) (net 8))
 (segment (start 126.492 124.714) (end 135.287 124.714) (width 0.762) (layer B.Cu) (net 8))
 (segment (start 123.317 121.539) (end 126.492 124.714) (width 0.762) (layer B.Cu) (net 8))
 (segment (start 135.2235 124.6505) (end 135.287 124.714) (width 0.762) (layer B.Cu) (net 8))
 (segment (start 137.066 128.016) (end 137.066 131.605) (width 0.3048) (layer F.Cu) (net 9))
 (segment (start 137.922 129.159) (end 139.287 129.159) (width 0.3048) (layer B.Cu) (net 9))
 (segment (start 137.541 129.54) (end 137.922 129.159) (width 0.3048) (layer B.Cu) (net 9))
 (segment (start 137.541 131.318) (end 137.541 129.54) (width 0.3048) (layer B.Cu) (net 9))
 (segment (start 137.16 131.699) (end 137.541 131.318) (width 0.3048) (layer B.Cu) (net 9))
 (via (at 137.16 131.699) (size 1.27) (drill 0.7112) (layers F.Cu B.Cu) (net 9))
 (segment (start 137.066 131.605) (end 137.16 131.699) (width 0.3048) (layer F.Cu) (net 9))
 (segment (start 139.287 124.714) (end 139.287 129.159) (width 0.762) (layer B.Cu) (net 9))
 (segment (start 131.666 120.302) (end 131.666 124.206) (width 0.3048) (layer F.Cu) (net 10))
 (segment (start 131.953 120.015) (end 131.666 120.302) (width 0.3048) (layer F.Cu) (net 10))
 (via (at 131.953 120.015) (size 1.27) (drill 0.7112) (layers F.Cu B.Cu) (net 10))
 (segment (start 142.748 120.015) (end 131.953 120.015) (width 0.3048) (layer B.Cu) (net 10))
 (via (at 142.748 120.015) (size 1.27) (drill 0.7112) (layers F.Cu B.Cu) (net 10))
 (segment (start 142.748 124.206) (end 142.748 120.015) (width 0.3048) (layer F.Cu) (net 10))
 (via (at 142.748 124.206) (size 1.27) (drill 0.7112) (layers F.Cu B.Cu) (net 10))
 (segment (start 142.875 124.079) (end 142.748 124.206) (width 0.3048) (layer B.Cu) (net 10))
 (segment (start 146.685 124.079) (end 142.875 124.079) (width 0.3048) (layer B.Cu) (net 10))
 (segment (start 131.666 128.016) (end 133.096 128.016) (width 0.3048) (layer F.Cu) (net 11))
 (segment (start 141.859 121.539) (end 141.351 121.031) (width 0.3048) (layer B.Cu) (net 11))
 (segment (start 141.351 121.031) (end 134.366 121.031) (width 0.3048) (layer B.Cu) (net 11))
 (segment (start 134.366 121.031) (end 133.477 122.301) (width 0.3048) (layer B.Cu) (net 11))
 (via (at 133.477 122.301) (size 1.27) (drill 0.7112) (layers F.Cu B.Cu) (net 11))
 (segment (start 133.477 122.301) (end 133.604 122.809) (width 0.3048) (layer F.Cu) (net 11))
 (segment (start 133.604 122.809) (end 133.604 127.508) (width 0.3048) (layer F.Cu) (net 11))
 (segment (start 133.604 127.508) (end 133.096 128.016) (width 0.3048) (layer F.Cu) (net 11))
 (segment (start 141.859 121.539) (end 146.685 121.539) (width 0.3048) (layer B.Cu) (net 11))
 (segment (start 139.192 114.554) (end 137.34542 114.554) (width 0.3048) (layer F.Cu) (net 18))
 (segment (start 139.954 115.316) (end 139.192 114.554) (width 0.3048) (layer F.Cu) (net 18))
 (segment (start 139.954 131.572) (end 139.954 115.316) (width 0.3048) (layer F.Cu) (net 18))
 (segment (start 140.081 131.699) (end 139.954 131.572) (width 0.3048) (layer B.Cu) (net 18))
 (via (at 139.954 131.572) (size 1.27) (drill 0.7112) (layers F.Cu B.Cu) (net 18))
 (segment (start 146.685 131.699) (end 140.081 131.699) (width 0.3048) (layer B.Cu) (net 18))
 (segment (start 146.685 134.239) (end 141.859 134.239) (width 0.3048) (layer B.Cu) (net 19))
 (segment (start 139.827 113.284) (end 137.34542 113.284) (width 0.3048) (layer F.Cu) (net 19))
 (segment (start 141.351 114.808) (end 139.827 113.284) (width 0.3048) (layer F.Cu) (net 19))
 (segment (start 141.351 133.731) (end 141.351 114.808) (width 0.3048) (layer F.Cu) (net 19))
 (segment (start 141.859 134.239) (end 141.351 133.731) (width 0.3048) (layer F.Cu) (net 19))
 (via (at 141.859 134.239) (size 1.27) (drill 0.7112) (layers F.Cu B.Cu) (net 19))
 (segment (start 137.34542 112.014) (end 141.732 112.014) (width 0.3048) (layer F.Cu) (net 20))
 (segment (start 143.637 118.999) (end 146.685 118.999) (width 0.3048) (layer F.Cu) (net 20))
 (segment (start 142.748 118.11) (end 143.637 118.999) (width 0.3048) (layer F.Cu) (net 20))
 (segment (start 142.748 113.03) (end 142.748 118.11) (width 0.3048) (layer F.Cu) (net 20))
 (segment (start 141.732 112.014) (end 142.748 113.03) (width 0.3048) (layer F.Cu) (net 20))
 (segment (start 146.685 116.459) (end 144.78 116.459) (width 0.3048) (layer F.Cu) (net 21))
 (segment (start 142.748 110.744) (end 137.34542 110.744) (width 0.3048) (layer F.Cu) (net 21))
 (segment (start 143.891 111.887) (end 142.748 110.744) (width 0.3048) (layer F.Cu) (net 21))
 (segment (start 143.891 115.57) (end 143.891 111.887) (width 0.3048) (layer F.Cu) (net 21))
 (segment (start 144.78 116.459) (end 143.891 115.57) (width 0.3048) (layer F.Cu) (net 21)))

